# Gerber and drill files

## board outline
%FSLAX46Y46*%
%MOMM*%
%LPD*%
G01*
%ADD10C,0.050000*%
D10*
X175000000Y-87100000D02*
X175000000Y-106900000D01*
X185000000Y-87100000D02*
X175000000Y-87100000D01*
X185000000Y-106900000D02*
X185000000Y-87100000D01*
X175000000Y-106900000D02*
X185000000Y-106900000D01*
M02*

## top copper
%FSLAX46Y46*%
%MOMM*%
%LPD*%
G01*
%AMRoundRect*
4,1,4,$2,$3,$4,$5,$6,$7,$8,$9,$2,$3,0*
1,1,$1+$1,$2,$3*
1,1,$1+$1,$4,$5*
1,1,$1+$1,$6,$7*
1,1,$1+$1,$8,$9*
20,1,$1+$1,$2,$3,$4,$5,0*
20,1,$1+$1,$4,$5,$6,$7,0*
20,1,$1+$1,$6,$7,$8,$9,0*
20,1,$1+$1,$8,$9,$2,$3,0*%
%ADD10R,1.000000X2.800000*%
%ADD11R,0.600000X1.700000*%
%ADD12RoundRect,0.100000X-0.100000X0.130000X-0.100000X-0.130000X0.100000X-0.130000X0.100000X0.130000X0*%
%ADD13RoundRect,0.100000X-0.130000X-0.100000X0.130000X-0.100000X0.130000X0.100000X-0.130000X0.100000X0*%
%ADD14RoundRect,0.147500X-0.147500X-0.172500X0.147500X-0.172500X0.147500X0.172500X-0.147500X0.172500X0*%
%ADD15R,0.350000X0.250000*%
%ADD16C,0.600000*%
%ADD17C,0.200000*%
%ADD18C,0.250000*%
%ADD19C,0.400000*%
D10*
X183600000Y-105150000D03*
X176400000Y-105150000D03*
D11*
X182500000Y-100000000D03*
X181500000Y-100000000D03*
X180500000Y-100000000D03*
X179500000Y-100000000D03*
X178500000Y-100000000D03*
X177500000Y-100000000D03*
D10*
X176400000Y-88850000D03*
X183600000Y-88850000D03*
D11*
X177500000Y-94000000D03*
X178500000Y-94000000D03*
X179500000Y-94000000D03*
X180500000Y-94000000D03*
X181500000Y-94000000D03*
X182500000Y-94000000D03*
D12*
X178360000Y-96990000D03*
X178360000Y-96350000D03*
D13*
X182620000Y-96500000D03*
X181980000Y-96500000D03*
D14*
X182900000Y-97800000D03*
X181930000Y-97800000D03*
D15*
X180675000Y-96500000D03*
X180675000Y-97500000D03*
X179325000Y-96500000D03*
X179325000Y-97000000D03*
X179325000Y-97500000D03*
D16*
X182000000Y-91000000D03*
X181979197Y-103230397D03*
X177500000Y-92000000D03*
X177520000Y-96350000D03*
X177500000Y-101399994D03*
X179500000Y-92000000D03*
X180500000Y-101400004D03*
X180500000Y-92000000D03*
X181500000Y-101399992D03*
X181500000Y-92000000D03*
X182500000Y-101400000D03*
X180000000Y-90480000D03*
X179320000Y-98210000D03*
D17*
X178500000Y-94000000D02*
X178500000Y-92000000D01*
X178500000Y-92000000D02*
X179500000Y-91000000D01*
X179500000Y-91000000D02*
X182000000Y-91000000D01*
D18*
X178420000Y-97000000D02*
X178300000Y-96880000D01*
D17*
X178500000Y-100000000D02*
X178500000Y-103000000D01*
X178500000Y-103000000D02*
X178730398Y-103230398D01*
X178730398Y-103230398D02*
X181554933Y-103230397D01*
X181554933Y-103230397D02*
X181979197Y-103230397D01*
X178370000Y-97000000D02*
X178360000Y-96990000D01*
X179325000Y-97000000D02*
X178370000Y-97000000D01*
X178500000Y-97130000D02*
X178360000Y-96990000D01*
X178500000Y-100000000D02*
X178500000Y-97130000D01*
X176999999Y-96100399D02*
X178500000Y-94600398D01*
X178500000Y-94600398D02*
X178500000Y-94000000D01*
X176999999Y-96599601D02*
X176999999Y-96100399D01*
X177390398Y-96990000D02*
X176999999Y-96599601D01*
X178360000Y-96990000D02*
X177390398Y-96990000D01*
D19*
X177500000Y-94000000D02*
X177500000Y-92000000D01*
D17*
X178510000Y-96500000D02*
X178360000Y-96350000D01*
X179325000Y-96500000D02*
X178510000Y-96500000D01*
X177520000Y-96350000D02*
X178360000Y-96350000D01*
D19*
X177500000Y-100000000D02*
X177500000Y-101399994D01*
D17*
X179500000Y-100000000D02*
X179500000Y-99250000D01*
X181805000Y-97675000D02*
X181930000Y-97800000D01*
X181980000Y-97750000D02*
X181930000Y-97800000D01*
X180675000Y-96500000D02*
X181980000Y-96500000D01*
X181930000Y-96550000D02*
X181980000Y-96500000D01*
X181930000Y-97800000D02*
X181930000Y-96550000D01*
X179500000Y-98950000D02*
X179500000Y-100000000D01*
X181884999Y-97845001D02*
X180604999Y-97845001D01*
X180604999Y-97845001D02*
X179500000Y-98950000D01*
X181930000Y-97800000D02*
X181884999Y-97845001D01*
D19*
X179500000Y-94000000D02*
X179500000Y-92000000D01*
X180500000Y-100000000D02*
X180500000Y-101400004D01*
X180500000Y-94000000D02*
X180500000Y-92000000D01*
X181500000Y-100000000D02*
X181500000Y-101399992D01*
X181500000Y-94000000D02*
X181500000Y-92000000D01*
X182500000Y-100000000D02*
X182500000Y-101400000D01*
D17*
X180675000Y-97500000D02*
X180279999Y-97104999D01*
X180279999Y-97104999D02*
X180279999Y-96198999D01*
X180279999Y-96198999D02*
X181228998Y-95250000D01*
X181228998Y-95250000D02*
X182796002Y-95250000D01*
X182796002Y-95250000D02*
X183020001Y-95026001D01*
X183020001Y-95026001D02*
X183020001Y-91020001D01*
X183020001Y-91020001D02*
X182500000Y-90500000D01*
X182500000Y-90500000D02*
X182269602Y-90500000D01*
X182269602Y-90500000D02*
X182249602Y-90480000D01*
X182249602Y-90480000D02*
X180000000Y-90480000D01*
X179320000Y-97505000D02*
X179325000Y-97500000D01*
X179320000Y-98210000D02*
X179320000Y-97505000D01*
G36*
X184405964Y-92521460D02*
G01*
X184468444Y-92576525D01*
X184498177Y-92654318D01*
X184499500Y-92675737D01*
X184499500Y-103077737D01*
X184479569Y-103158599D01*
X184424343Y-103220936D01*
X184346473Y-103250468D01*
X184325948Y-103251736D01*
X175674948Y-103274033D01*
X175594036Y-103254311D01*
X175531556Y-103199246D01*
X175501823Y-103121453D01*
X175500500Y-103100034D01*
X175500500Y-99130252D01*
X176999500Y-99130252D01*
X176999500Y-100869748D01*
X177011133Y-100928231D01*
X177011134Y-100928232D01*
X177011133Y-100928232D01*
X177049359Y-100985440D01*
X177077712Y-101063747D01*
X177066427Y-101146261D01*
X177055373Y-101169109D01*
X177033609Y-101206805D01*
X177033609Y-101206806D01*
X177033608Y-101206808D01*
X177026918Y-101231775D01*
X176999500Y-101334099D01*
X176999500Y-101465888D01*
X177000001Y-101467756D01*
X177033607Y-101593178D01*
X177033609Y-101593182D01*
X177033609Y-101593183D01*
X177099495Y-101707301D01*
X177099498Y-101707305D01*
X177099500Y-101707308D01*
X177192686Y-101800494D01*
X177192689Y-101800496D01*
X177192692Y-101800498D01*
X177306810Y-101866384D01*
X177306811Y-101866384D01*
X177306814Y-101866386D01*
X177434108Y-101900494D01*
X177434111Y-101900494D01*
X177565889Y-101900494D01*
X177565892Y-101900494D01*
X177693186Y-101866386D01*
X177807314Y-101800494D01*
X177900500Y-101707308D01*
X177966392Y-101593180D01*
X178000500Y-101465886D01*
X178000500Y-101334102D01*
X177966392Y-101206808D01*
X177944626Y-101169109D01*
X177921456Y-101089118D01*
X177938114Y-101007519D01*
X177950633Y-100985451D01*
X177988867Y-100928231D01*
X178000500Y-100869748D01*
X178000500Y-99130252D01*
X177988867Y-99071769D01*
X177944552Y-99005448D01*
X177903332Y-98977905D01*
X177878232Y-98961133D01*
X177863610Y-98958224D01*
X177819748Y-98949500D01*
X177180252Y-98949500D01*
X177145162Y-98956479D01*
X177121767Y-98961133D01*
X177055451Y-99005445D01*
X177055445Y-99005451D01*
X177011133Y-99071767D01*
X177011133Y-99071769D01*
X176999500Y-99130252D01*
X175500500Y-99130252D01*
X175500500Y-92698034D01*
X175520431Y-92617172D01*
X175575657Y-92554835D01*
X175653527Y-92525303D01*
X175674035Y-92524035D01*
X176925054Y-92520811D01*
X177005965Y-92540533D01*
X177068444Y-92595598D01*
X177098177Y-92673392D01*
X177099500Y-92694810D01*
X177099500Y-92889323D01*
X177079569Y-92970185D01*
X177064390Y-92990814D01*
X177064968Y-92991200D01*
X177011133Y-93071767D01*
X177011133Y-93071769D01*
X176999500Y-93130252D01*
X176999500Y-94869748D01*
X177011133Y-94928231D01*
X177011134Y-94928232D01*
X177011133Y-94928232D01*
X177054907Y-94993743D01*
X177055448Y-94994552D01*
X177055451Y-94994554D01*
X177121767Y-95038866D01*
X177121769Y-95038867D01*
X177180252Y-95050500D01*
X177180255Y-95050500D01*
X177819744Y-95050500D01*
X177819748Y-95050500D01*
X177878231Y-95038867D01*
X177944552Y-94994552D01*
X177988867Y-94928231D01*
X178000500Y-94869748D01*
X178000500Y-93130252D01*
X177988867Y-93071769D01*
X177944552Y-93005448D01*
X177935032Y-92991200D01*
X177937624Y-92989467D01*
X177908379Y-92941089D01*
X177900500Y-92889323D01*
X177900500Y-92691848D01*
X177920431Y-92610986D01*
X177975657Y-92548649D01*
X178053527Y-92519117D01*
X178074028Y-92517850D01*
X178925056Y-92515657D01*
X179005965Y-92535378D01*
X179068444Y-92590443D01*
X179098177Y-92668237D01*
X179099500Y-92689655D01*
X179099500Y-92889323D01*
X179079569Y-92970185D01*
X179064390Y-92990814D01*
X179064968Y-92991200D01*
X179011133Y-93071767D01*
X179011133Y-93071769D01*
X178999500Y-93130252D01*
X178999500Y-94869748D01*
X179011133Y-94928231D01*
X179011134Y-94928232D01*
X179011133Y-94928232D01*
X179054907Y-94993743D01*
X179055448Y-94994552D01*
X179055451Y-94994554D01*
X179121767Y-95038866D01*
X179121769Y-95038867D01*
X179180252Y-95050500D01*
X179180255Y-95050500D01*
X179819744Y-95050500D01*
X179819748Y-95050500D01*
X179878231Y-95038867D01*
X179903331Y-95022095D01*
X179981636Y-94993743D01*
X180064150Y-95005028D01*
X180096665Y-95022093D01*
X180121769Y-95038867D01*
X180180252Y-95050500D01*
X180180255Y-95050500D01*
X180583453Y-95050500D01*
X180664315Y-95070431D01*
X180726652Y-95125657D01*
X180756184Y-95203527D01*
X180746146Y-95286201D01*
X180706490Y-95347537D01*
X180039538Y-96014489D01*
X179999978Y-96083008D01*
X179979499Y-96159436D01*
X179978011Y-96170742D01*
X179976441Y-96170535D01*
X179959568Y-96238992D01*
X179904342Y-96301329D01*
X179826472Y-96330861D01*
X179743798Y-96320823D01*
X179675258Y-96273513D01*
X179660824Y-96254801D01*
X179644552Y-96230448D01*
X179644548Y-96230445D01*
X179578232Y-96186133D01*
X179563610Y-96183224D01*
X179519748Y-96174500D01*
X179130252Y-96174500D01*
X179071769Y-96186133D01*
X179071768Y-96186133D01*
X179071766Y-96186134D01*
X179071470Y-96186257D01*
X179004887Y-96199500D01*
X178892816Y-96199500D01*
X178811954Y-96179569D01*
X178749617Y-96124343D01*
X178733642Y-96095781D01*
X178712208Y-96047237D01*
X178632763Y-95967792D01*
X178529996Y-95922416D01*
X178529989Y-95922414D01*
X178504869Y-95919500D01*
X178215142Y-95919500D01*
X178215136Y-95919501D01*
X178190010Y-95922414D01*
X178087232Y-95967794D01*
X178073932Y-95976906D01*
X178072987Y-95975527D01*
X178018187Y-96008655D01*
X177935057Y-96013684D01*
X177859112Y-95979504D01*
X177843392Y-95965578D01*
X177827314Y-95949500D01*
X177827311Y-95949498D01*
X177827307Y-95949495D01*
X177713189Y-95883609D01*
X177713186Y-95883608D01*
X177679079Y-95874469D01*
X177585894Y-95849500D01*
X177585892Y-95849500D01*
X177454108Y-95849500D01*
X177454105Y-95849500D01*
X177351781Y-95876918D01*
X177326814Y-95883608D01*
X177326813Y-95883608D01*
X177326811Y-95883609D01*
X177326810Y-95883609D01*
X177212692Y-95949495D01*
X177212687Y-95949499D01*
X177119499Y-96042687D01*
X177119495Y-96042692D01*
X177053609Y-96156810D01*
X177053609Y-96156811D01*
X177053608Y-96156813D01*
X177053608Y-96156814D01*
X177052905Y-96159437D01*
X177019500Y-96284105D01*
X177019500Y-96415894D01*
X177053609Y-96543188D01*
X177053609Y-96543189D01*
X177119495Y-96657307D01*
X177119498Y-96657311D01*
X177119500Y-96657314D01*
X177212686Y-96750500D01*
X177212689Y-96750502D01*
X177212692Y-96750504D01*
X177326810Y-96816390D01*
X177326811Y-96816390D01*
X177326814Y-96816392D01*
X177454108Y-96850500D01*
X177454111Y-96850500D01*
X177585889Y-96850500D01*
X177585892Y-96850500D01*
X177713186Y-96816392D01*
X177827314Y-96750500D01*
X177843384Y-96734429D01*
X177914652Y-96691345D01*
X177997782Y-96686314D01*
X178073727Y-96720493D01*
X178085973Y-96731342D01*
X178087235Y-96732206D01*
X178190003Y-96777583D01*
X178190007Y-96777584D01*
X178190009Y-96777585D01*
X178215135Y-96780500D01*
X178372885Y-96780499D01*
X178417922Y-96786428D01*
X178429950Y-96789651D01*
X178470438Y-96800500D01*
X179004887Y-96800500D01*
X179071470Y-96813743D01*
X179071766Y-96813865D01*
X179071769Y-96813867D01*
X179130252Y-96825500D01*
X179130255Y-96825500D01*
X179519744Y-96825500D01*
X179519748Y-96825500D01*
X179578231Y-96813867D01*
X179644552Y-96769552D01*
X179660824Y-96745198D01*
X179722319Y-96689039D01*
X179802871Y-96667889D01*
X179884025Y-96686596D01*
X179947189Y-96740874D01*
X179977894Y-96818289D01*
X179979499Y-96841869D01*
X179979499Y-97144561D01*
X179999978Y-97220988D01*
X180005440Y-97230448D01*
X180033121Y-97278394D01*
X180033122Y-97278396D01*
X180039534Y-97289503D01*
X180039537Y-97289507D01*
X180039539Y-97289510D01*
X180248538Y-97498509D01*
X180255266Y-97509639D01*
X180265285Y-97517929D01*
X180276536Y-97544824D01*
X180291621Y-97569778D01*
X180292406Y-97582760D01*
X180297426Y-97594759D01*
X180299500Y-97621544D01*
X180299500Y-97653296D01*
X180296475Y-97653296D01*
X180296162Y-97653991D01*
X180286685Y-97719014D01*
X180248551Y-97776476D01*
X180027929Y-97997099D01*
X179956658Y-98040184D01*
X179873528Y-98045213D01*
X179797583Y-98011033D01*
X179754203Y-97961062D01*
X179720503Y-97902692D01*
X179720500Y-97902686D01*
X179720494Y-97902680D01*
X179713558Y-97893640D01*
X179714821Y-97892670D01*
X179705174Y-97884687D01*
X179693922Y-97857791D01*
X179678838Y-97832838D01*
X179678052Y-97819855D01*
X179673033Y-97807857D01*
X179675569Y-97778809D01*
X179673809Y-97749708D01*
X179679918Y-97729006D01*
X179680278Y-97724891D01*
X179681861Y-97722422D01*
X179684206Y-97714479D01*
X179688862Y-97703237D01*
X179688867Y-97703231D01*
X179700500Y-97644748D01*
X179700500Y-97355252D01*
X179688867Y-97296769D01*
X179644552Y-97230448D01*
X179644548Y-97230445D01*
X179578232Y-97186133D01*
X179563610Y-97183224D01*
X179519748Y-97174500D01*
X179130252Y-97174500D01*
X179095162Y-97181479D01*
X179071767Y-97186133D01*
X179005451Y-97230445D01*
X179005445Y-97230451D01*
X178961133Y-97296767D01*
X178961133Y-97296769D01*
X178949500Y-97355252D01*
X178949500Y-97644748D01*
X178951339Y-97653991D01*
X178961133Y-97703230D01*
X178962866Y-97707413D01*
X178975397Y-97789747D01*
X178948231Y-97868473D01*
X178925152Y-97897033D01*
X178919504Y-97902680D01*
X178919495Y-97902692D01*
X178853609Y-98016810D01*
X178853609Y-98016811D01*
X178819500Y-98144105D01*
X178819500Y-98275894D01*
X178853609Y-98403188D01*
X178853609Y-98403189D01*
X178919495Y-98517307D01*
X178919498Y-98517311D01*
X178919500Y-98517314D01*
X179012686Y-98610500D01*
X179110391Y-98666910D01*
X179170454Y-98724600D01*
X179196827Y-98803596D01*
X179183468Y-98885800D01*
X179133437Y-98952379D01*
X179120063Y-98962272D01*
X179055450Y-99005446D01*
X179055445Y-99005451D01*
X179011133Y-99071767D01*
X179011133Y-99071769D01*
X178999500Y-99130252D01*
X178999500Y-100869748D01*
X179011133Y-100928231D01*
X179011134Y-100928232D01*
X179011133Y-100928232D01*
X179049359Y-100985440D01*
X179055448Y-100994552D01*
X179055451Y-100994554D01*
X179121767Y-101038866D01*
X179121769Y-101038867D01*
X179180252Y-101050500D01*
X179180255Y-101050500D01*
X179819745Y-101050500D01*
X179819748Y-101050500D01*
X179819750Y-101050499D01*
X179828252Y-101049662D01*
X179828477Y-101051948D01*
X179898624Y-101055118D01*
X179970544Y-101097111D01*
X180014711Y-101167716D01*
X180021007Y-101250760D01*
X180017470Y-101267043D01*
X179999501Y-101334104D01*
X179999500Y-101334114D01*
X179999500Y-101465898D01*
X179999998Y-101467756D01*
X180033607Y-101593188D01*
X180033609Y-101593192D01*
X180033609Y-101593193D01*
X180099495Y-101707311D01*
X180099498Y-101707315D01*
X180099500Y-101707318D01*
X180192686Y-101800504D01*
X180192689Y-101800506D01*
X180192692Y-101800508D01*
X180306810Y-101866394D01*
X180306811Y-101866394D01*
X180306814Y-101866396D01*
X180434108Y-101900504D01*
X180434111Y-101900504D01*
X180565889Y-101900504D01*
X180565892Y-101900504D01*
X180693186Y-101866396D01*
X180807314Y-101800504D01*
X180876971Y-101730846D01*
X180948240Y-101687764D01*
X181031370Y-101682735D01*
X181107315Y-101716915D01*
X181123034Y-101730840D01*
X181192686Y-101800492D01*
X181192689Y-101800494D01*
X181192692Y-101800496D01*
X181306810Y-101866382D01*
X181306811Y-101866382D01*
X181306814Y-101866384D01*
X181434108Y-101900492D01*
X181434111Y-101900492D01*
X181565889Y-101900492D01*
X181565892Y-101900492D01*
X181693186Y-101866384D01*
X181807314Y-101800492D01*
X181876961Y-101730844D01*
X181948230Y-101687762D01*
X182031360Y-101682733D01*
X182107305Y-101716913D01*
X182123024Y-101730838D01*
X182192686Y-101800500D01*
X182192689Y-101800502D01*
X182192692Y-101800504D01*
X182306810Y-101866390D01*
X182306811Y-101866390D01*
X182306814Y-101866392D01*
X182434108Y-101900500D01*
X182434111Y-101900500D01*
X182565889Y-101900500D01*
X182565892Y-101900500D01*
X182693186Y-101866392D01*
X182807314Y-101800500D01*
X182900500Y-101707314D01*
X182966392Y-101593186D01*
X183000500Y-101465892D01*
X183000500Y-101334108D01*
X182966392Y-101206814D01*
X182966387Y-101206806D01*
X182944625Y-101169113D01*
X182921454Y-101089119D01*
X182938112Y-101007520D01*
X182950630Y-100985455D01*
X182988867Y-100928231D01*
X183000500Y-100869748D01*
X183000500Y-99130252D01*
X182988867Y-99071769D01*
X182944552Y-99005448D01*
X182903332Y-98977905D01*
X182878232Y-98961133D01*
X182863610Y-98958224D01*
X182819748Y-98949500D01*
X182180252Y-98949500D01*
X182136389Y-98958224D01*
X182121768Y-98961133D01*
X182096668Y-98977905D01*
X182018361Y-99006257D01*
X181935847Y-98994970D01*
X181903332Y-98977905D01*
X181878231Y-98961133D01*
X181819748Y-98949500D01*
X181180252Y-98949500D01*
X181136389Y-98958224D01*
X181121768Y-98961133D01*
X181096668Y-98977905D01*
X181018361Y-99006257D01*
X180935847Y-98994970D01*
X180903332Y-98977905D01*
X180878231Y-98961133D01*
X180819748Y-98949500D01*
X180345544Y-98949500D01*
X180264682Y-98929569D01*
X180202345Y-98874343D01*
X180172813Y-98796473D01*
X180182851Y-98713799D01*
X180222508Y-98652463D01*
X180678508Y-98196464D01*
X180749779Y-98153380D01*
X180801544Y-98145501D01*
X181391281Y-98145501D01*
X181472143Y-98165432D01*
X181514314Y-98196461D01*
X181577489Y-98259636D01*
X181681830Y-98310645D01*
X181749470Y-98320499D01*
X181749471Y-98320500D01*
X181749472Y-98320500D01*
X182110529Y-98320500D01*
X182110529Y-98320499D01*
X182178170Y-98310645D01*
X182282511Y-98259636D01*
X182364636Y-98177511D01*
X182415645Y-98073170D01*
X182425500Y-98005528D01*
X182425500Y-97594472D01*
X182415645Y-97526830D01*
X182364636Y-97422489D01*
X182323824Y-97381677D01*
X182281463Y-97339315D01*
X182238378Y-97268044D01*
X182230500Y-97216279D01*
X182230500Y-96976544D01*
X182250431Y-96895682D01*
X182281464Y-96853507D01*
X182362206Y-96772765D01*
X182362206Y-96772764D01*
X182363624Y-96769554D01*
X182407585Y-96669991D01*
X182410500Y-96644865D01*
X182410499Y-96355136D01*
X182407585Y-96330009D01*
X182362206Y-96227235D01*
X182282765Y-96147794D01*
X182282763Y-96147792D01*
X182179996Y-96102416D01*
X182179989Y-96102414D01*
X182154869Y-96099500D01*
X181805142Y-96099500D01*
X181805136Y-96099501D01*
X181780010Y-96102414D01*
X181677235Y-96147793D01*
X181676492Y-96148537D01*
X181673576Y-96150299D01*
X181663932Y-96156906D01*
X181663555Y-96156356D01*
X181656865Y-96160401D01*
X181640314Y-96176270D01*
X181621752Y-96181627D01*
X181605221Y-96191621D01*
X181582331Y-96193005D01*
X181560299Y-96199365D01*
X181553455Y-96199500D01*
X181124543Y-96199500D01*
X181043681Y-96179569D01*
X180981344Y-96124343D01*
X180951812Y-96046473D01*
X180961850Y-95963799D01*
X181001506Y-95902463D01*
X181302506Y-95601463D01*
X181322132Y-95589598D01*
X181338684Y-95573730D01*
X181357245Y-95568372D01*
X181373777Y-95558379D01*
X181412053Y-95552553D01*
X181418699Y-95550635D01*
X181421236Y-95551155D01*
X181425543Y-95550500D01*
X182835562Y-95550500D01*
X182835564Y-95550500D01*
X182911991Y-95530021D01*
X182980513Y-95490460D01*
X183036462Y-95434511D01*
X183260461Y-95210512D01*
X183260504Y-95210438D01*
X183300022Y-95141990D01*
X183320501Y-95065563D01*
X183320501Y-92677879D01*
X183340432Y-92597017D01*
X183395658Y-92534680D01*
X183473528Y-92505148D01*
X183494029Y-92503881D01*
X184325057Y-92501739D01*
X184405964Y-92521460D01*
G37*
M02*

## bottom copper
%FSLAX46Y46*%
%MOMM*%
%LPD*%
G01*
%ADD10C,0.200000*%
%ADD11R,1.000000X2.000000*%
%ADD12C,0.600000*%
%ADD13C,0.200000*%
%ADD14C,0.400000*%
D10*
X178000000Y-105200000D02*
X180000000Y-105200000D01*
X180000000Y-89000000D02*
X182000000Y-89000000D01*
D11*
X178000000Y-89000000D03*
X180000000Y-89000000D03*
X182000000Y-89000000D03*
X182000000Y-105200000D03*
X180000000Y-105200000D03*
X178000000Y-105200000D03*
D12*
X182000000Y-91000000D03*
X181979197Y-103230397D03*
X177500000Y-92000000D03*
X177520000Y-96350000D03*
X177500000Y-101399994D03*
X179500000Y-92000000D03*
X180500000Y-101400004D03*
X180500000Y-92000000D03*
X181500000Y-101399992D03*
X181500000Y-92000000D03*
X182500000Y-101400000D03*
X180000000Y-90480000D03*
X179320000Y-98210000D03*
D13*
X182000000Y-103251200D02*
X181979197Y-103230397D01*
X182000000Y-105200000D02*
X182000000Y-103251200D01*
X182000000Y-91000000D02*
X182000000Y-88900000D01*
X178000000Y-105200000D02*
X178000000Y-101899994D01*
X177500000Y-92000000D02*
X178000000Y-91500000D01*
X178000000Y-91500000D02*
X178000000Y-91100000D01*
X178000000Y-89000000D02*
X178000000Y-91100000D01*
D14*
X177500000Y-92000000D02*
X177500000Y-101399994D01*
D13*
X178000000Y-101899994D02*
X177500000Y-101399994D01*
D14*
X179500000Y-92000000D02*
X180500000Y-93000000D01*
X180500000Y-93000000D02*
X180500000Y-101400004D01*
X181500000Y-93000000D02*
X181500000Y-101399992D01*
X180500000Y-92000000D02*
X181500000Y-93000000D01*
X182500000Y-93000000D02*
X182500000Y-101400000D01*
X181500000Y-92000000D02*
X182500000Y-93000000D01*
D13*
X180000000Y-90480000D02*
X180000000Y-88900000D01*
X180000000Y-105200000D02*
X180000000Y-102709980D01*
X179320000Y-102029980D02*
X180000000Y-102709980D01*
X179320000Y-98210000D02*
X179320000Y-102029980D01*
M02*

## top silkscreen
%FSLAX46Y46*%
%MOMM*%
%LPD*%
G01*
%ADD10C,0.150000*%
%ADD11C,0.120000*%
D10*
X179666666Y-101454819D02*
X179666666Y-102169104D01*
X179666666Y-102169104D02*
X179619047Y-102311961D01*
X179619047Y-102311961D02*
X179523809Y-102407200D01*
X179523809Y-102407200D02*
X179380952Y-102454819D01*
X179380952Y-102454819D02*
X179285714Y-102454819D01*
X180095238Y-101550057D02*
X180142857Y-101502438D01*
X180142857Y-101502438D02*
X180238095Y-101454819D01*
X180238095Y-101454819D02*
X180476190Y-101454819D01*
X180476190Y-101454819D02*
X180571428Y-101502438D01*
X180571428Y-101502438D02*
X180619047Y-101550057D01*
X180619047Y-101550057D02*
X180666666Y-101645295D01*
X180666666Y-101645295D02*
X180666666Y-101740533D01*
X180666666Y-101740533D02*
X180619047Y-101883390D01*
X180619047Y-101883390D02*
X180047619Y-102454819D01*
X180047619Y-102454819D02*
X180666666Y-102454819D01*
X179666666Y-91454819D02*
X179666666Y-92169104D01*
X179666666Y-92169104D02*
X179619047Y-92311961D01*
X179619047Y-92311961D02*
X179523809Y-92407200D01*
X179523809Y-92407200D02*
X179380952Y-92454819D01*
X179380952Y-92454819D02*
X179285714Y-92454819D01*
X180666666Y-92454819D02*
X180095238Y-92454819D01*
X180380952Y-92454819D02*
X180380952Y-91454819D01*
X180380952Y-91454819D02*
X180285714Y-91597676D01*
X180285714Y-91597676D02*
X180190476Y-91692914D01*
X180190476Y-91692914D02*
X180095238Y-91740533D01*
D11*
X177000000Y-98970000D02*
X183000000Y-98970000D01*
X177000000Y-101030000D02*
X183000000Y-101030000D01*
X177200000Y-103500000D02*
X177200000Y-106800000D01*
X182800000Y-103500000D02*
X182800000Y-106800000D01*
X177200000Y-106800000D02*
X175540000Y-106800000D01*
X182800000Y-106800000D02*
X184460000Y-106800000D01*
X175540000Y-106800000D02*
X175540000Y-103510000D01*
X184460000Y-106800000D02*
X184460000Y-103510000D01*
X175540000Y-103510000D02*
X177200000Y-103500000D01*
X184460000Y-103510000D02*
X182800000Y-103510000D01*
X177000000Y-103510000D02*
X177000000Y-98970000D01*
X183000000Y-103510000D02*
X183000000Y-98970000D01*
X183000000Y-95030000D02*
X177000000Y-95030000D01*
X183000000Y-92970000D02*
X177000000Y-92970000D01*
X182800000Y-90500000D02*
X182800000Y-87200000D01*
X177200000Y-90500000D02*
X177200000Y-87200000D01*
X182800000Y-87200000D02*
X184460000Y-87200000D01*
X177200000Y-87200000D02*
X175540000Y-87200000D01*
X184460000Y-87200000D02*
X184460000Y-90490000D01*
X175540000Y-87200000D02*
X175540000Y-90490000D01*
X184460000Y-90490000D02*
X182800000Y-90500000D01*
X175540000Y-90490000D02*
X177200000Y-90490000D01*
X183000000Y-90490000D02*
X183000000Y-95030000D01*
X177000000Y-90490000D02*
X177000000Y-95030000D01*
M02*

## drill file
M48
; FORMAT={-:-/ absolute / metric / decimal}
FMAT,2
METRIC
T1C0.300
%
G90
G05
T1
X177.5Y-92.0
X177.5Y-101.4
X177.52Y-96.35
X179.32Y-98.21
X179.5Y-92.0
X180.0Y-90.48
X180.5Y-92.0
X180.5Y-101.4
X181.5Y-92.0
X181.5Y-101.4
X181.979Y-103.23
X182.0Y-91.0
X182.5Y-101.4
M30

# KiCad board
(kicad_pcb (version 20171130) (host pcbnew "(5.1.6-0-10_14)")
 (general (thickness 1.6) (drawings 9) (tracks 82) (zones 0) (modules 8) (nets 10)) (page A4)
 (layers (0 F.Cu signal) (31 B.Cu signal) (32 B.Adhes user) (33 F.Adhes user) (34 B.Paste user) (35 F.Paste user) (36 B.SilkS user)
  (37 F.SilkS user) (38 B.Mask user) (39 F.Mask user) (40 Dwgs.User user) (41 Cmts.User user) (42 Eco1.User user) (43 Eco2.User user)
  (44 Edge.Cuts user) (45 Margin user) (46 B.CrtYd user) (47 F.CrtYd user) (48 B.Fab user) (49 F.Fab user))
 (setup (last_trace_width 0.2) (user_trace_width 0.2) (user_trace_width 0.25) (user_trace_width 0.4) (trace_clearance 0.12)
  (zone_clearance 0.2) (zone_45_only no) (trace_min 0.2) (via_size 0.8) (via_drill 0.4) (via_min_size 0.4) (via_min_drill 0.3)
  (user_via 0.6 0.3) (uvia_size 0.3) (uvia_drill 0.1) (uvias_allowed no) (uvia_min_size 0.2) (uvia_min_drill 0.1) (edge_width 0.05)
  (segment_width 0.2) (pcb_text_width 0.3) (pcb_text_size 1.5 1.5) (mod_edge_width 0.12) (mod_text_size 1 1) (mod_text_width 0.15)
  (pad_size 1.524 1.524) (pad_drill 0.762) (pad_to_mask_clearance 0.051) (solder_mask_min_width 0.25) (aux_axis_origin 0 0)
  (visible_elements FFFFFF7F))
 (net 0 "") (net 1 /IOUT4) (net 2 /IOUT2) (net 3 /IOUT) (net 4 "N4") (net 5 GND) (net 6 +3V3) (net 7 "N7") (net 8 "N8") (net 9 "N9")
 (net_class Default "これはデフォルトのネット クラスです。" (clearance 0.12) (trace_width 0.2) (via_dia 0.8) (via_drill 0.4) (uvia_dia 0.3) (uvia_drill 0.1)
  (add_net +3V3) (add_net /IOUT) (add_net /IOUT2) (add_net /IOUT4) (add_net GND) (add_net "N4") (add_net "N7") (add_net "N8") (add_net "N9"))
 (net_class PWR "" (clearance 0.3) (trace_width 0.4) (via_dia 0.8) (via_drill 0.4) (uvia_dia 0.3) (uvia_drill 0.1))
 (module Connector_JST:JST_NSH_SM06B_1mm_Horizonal (layer F.Cu) (at 180 100)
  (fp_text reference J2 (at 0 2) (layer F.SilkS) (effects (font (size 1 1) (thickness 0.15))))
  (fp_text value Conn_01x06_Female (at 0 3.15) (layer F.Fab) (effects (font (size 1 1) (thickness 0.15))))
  (fp_line (start -3 -1.03) (end 3 -1.03) (layer F.SilkS) (width 0.12))
  (fp_line (start -3 1.03) (end 3 1.03) (layer F.SilkS) (width 0.12))
  (fp_line (start -2.8 3.5) (end -2.8 6.8) (layer F.SilkS) (width 0.12))
  (fp_line (start 2.8 3.5) (end 2.8 6.8) (layer F.SilkS) (width 0.12))
  (fp_line (start -2.8 6.8) (end -4.46 6.8) (layer F.SilkS) (width 0.12))
  (fp_line (start 2.8 6.8) (end 4.46 6.8) (layer F.SilkS) (width 0.12))
  (fp_line (start -4.46 6.8) (end -4.46 3.51) (layer F.SilkS) (width 0.12))
  (fp_line (start 4.46 6.8) (end 4.46 3.51) (layer F.SilkS) (width 0.12))
  (fp_line (start -4.46 3.51) (end -2.8 3.5) (layer F.SilkS) (width 0.12))
  (fp_line (start 4.46 3.51) (end 2.8 3.51) (layer F.SilkS) (width 0.12))
  (fp_line (start -3 3.51) (end -3 -1.03) (layer F.SilkS) (width 0.12))
  (fp_line (start 3 3.51) (end 3 -1.03) (layer F.SilkS) (width 0.12))
  (pad 0 smd rect (at 3.6 5.15) (size 1 2.8) (layers F.Cu F.Paste F.Mask))
  (pad 0 smd rect (at -3.6 5.15) (size 1 2.8) (layers F.Cu F.Paste F.Mask))
  (pad 6 smd rect (at 2.5 0) (size 0.6 1.7) (layers F.Cu F.Paste F.Mask) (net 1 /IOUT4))
  (pad 5 smd rect (at 1.5 0) (size 0.6 1.7) (layers F.Cu F.Paste F.Mask) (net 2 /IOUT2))
  (pad 4 smd rect (at 0.5 0) (size 0.6 1.7) (layers F.Cu F.Paste F.Mask) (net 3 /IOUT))
  (pad 3 smd rect (at -0.5 0) (size 0.6 1.7) (layers F.Cu F.Paste F.Mask) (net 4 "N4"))
  (pad 2 smd rect (at -1.5 0) (size 0.6 1.7) (layers F.Cu F.Paste F.Mask) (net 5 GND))
  (pad 1 smd rect (at -2.5 0) (size 0.6 1.7) (layers F.Cu F.Paste F.Mask) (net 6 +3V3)))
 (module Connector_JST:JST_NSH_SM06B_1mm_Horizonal (layer F.Cu) (at 180 94 180)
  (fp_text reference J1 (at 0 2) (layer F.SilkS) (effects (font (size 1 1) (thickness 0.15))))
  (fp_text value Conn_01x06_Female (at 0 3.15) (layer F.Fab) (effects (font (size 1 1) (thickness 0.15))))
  (fp_line (start -3 -1.03) (end 3 -1.03) (layer F.SilkS) (width 0.12))
  (fp_line (start -3 1.03) (end 3 1.03) (layer F.SilkS) (width 0.12))
  (fp_line (start -2.8 3.5) (end -2.8 6.8) (layer F.SilkS) (width 0.12))
  (fp_line (start 2.8 3.5) (end 2.8 6.8) (layer F.SilkS) (width 0.12))
  (fp_line (start -2.8 6.8) (end -4.46 6.8) (layer F.SilkS) (width 0.12))
  (fp_line (start 2.8 6.8) (end 4.46 6.8) (layer F.SilkS) (width 0.12))
  (fp_line (start -4.46 6.8) (end -4.46 3.51) (layer F.SilkS) (width 0.12))
  (fp_line (start 4.46 6.8) (end 4.46 3.51) (layer F.SilkS) (width 0.12))
  (fp_line (start -4.46 3.51) (end -2.8 3.5) (layer F.SilkS) (width 0.12))
  (fp_line (start 4.46 3.51) (end 2.8 3.51) (layer F.SilkS) (width 0.12))
  (fp_line (start -3 3.51) (end -3 -1.03) (layer F.SilkS) (width 0.12))
  (fp_line (start 3 3.51) (end 3 -1.03) (layer F.SilkS) (width 0.12))
  (pad 0 smd rect (at 3.6 5.15 180) (size 1 2.8) (layers F.Cu F.Paste F.Mask))
  (pad 0 smd rect (at -3.6 5.15 180) (size 1 2.8) (layers F.Cu F.Paste F.Mask))
  (pad 6 smd rect (at 2.5 0 180) (size 0.6 1.7) (layers F.Cu F.Paste F.Mask) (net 6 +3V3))
  (pad 5 smd rect (at 1.5 0 180) (size 0.6 1.7) (layers F.Cu F.Paste F.Mask) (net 5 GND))
  (pad 4 smd rect (at 0.5 0 180) (size 0.6 1.7) (layers F.Cu F.Paste F.Mask) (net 3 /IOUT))
  (pad 3 smd rect (at -0.5 0 180) (size 0.6 1.7) (layers F.Cu F.Paste F.Mask) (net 2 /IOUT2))
  (pad 2 smd rect (at -1.5 0 180) (size 0.6 1.7) (layers F.Cu F.Paste F.Mask) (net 1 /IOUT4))
  (pad 1 smd rect (at -2.5 0 180) (size 0.6 1.7) (layers F.Cu F.Paste F.Mask) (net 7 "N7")))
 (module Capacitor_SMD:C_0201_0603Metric (layer F.Cu) (at 178.36 96.67 270)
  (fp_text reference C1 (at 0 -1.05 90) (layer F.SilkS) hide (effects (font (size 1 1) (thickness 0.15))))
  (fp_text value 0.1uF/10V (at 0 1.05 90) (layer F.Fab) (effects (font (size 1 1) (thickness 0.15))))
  (pad 2 smd roundrect (at 0.32 0 270) (size 0.46 0.4) (layers F.Cu F.Mask) (roundrect_rratio 0.25) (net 5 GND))
  (pad 1 smd roundrect (at -0.32 0 270) (size 0.46 0.4) (layers F.Cu F.Mask) (roundrect_rratio 0.25) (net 6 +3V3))
  (pad "" smd roundrect (at 0.345 0 270) (size 0.318 0.36) (layers F.Paste) (roundrect_rratio 0.25))
  (pad "" smd roundrect (at -0.345 0 270) (size 0.318 0.36) (layers F.Paste) (roundrect_rratio 0.25)))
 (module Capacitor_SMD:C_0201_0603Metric (layer F.Cu) (at 182.3 96.5)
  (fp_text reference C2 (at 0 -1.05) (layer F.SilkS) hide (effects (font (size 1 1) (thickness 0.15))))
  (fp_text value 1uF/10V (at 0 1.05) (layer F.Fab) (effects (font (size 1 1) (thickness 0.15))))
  (pad 2 smd roundrect (at 0.32 0) (size 0.46 0.4) (layers F.Cu F.Mask) (roundrect_rratio 0.25) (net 5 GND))
  (pad 1 smd roundrect (at -0.32 0) (size 0.46 0.4) (layers F.Cu F.Mask) (roundrect_rratio 0.25) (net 4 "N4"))
  (pad "" smd roundrect (at 0.345 0) (size 0.318 0.36) (layers F.Paste) (roundrect_rratio 0.25))
  (pad "" smd roundrect (at -0.345 0) (size 0.318 0.36) (layers F.Paste) (roundrect_rratio 0.25)))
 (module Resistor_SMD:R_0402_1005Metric (layer F.Cu) (at 182.415 97.8)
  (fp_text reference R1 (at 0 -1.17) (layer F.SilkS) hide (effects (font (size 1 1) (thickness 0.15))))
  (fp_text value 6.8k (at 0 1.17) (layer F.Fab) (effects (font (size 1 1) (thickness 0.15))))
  (pad 2 smd roundrect (at 0.485 0) (size 0.59 0.64) (layers F.Cu F.Paste F.Mask) (roundrect_rratio 0.25) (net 5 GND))
  (pad 1 smd roundrect (at -0.485 0) (size 0.59 0.64) (layers F.Cu F.Paste F.Mask) (roundrect_rratio 0.25) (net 4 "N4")))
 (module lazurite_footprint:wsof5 (layer F.Cu) (at 180.5 97 90)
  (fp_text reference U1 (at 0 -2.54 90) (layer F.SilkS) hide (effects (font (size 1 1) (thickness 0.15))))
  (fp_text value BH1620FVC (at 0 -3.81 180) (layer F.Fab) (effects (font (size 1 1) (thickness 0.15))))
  (pad 5 smd rect (at 0.5 0.175 90) (size 0.25 0.35) (layers F.Cu F.Paste F.Mask) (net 4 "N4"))
  (pad 4 smd rect (at -0.5 0.175 90) (size 0.25 0.35) (layers F.Cu F.Paste F.Mask) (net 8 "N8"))
  (pad 1 smd rect (at 0.5 -1.175 90) (size 0.25 0.35) (layers F.Cu F.Paste F.Mask) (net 6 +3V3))
  (pad 2 smd rect (at 0 -1.175 90) (size 0.25 0.35) (layers F.Cu F.Paste F.Mask) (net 5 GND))
  (pad 3 smd rect (at -0.5 -1.175 90) (size 0.25 0.35) (layers F.Cu F.Paste F.Mask) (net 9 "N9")))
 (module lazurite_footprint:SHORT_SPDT (layer B.Cu) (at 180 89 270)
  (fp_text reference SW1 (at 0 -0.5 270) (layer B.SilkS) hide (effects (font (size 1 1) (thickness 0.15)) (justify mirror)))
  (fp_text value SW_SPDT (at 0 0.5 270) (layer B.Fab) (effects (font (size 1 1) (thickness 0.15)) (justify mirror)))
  (pad 3 smd rect (at 0 2 270) (size 2 1) (layers B.Cu B.Paste B.Mask) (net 6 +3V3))
  (pad 2 smd rect (at 0 0 270) (size 2 1) (layers B.Cu B.Paste B.Mask) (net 8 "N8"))
  (pad 1 smd rect (at 0 -2 270) (size 2 1) (layers B.Cu B.Paste B.Mask) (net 5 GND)))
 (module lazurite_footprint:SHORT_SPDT (layer B.Cu) (at 180 105.2 90)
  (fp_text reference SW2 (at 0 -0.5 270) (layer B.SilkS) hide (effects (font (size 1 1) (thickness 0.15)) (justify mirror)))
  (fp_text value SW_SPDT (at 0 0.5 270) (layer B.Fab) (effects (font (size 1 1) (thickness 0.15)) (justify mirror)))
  (pad 3 smd rect (at 0 2 90) (size 2 1) (layers B.Cu B.Paste B.Mask) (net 5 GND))
  (pad 2 smd rect (at 0 0 90) (size 2 1) (layers B.Cu B.Paste B.Mask) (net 9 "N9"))
  (pad 1 smd rect (at 0 -2 90) (size 2 1) (layers B.Cu B.Paste B.Mask) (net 6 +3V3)))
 (gr_line (start 178 105.2) (end 180 105.2) (layer B.Cu) (width 0.2))
 (gr_line (start 180 89) (end 182 89) (layer B.Cu) (width 0.2))
 (gr_line (start 175 87.1) (end 175 106.9) (layer Edge.Cuts) (width 0.05))
 (gr_line (start 185 87.1) (end 175 87.1) (layer Edge.Cuts) (width 0.05))
 (gr_line (start 185 106.9) (end 185 87.1) (layer Edge.Cuts) (width 0.05))
 (gr_line (start 175 106.9) (end 185 106.9) (layer Edge.Cuts) (width 0.05))
 (segment (start 178.5 94) (end 178.5 92) (width 0.2) (layer F.Cu) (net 5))
 (segment (start 178.5 92) (end 179.5 91) (width 0.2) (layer F.Cu) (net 5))
 (via (at 182 91) (size 0.6) (drill 0.3) (layers F.Cu B.Cu) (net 5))
 (segment (start 179.5 91) (end 182 91) (width 0.2) (layer F.Cu) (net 5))
 (segment (start 178.42 97) (end 178.3 96.88) (width 0.25) (layer F.Cu) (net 5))
 (via (at 181.979197 103.230397) (size 0.6) (drill 0.3) (layers F.Cu B.Cu) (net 5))
 (segment (start 178.5 100) (end 178.5 103) (width 0.2) (layer F.Cu) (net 5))
 (segment (start 178.5 103) (end 178.730398 103.230398) (width 0.2) (layer F.Cu) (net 5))
 (segment (start 178.730398 103.230398) (end 181.554933 103.230397) (width 0.2) (layer F.Cu) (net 5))
 (segment (start 181.554933 103.230397) (end 181.979197 103.230397) (width 0.2) (layer F.Cu) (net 5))
 (segment (start 182 103.2512) (end 181.979197 103.230397) (width 0.2) (layer B.Cu) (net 5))
 (segment (start 182 105.2) (end 182 103.2512) (width 0.2) (layer B.Cu) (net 5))
 (segment (start 182 91) (end 182 88.9) (width 0.2) (layer B.Cu) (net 5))
 (segment (start 178.37 97) (end 178.36 96.99) (width 0.2) (layer F.Cu) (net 5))
 (segment (start 179.325 97) (end 178.37 97) (width 0.2) (layer F.Cu) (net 5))
 (segment (start 178.5 97.13) (end 178.36 96.99) (width 0.2) (layer F.Cu) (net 5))
 (segment (start 178.5 100) (end 178.5 97.13) (width 0.2) (layer F.Cu) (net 5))
 (segment (start 176.999999 96.100399) (end 178.5 94.600398) (width 0.2) (layer F.Cu) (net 5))
 (segment (start 178.5 94.600398) (end 178.5 94) (width 0.2) (layer F.Cu) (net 5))
 (segment (start 176.999999 96.599601) (end 176.999999 96.100399) (width 0.2) (layer F.Cu) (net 5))
 (segment (start 177.390398 96.99) (end 176.999999 96.599601) (width 0.2) (layer F.Cu) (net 5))
 (segment (start 178.36 96.99) (end 177.390398 96.99) (width 0.2) (layer F.Cu) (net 5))
 (segment (start 177.5 94) (end 177.5 92) (width 0.4) (layer F.Cu) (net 6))
 (via (at 177.5 92) (size 0.6) (drill 0.3) (layers F.Cu B.Cu) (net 6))
 (via (at 177.52 96.35) (size 0.6) (drill 0.3) (layers F.Cu B.Cu) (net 6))
 (via (at 177.5 101.399994) (size 0.6) (drill 0.3) (layers F.Cu B.Cu) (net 6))
 (segment (start 178 105.2) (end 178 101.899994) (width 0.2) (layer B.Cu) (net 6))
 (segment (start 177.5 92) (end 178 91.5) (width 0.2) (layer B.Cu) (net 6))
 (segment (start 178 91.5) (end 178 91.1) (width 0.2) (layer B.Cu) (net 6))
 (segment (start 178 89) (end 178 91.1) (width 0.2) (layer B.Cu) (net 6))
 (segment (start 177.5 92) (end 177.5 101.399994) (width 0.4) (layer B.Cu) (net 6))
 (segment (start 178.51 96.5) (end 178.36 96.35) (width 0.2) (layer F.Cu) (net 6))
 (segment (start 179.325 96.5) (end 178.51 96.5) (width 0.2) (layer F.Cu) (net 6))
 (segment (start 178 101.899994) (end 177.5 101.399994) (width 0.2) (layer B.Cu) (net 6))
 (segment (start 177.52 96.35) (end 178.36 96.35) (width 0.2) (layer F.Cu) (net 6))
 (segment (start 177.5 100) (end 177.5 101.399994) (width 0.4) (layer F.Cu) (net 6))
 (segment (start 179.5 100) (end 179.5 99.25) (width 0.2) (layer F.Cu) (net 4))
 (segment (start 181.805 97.675) (end 181.93 97.8) (width 0.2) (layer F.Cu) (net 4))
 (segment (start 181.98 97.75) (end 181.93 97.8) (width 0.2) (layer F.Cu) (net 4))
 (segment (start 180.675 96.5) (end 181.98 96.5) (width 0.2) (layer F.Cu) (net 4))
 (segment (start 181.93 96.55) (end 181.98 96.5) (width 0.2) (layer F.Cu) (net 4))
 (segment (start 181.93 97.8) (end 181.93 96.55) (width 0.2) (layer F.Cu) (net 4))
 (segment (start 179.5 98.95) (end 179.5 100) (width 0.2) (layer F.Cu) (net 4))
 (segment (start 181.884999 97.845001) (end 180.604999 97.845001) (width 0.2) (layer F.Cu) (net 4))
 (segment (start 180.604999 97.845001) (end 179.5 98.95) (width 0.2) (layer F.Cu) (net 4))
 (segment (start 181.93 97.8) (end 181.884999 97.845001) (width 0.2) (layer F.Cu) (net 4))
 (segment (start 179.5 94) (end 179.5 92) (width 0.4) (layer F.Cu) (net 3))
 (via (at 179.5 92) (size 0.6) (drill 0.3) (layers F.Cu B.Cu) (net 3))
 (via (at 180.5 101.400004) (size 0.6) (drill 0.3) (layers F.Cu B.Cu) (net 3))
 (segment (start 179.5 92) (end 180.5 93) (width 0.4) (layer B.Cu) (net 3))
 (segment (start 180.5 100) (end 180.5 101.400004) (width 0.4) (layer F.Cu) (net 3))
 (segment (start 180.5 93) (end 180.5 101.400004) (width 0.4) (layer B.Cu) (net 3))
 (segment (start 180.5 94) (end 180.5 92) (width 0.4) (layer F.Cu) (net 2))
 (via (at 180.5 92) (size 0.6) (drill 0.3) (layers F.Cu B.Cu) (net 2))
 (segment (start 181.5 100) (end 181.5 101.399992) (width 0.4) (layer F.Cu) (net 2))
 (segment (start 181.5 93) (end 181.5 101.399992) (width 0.4) (layer B.Cu) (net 2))
 (via (at 181.5 101.399992) (size 0.6) (drill 0.3) (layers F.Cu B.Cu) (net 2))
 (segment (start 180.5 92) (end 181.5 93) (width 0.4) (layer B.Cu) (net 2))
 (segment (start 181.5 94) (end 181.5 92) (width 0.4) (layer F.Cu) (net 1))
 (via (at 181.5 92) (size 0.6) (drill 0.3) (layers F.Cu B.Cu) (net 1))
 (segment (start 182.5 93) (end 182.5 101.4) (width 0.4) (layer B.Cu) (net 1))
 (segment (start 181.5 92) (end 182.5 93) (width 0.4) (layer B.Cu) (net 1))
 (via (at 182.5 101.4) (size 0.6) (drill 0.3) (layers F.Cu B.Cu) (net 1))
 (segment (start 182.5 100) (end 182.5 101.4) (width 0.4) (layer F.Cu) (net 1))
 (via (at 180 90.48) (size 0.6) (drill 0.3) (layers F.Cu B.Cu) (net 8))
 (segment (start 180 90.48) (end 180 88.9) (width 0.2) (layer B.Cu) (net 8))
 (segment (start 180.675 97.5) (end 180.279999 97.104999) (width 0.2) (layer F.Cu) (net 8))
 (segment (start 180.279999 97.104999) (end 180.279999 96.198999) (width 0.2) (layer F.Cu) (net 8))
 (segment (start 180.279999 96.198999) (end 181.228998 95.25) (width 0.2) (layer F.Cu) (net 8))
 (segment (start 181.228998 95.25) (end 182.796002 95.25) (width 0.2) (layer F.Cu) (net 8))
 (segment (start 182.796002 95.25) (end 183.020001 95.026001) (width 0.2) (layer F.Cu) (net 8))
 (segment (start 183.020001 95.026001) (end 183.020001 91.020001) (width 0.2) (layer F.Cu) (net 8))
 (segment (start 183.020001 91.020001) (end 182.5 90.5) (width 0.2) (layer F.Cu) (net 8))
 (segment (start 182.5 90.5) (end 182.269602 90.5) (width 0.2) (layer F.Cu) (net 8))
 (segment (start 182.269602 90.5) (end 182.249602 90.48) (width 0.2) (layer F.Cu) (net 8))
 (segment (start 182.249602 90.48) (end 180 90.48) (width 0.2) (layer F.Cu) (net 8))
 (segment (start 180 105.2) (end 180 102.70998) (width 0.2) (layer B.Cu) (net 9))
 (via (at 179.32 98.21) (size 0.6) (drill 0.3) (layers F.Cu B.Cu) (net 9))
 (segment (start 179.32 97.505) (end 179.325 97.5) (width 0.2) (layer F.Cu) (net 9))
 (segment (start 179.32 102.02998) (end 180 102.70998) (width 0.2) (layer B.Cu) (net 9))
 (segment (start 179.32 98.21) (end 179.32 102.02998) (width 0.2) (layer B.Cu) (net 9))
 (segment (start 179.32 98.21) (end 179.32 97.505) (width 0.2) (layer F.Cu) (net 9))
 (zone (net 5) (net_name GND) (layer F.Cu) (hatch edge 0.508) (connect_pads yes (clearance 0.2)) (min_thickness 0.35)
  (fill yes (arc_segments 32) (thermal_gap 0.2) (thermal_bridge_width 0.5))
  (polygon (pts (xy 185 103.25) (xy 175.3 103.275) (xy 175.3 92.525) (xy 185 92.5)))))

